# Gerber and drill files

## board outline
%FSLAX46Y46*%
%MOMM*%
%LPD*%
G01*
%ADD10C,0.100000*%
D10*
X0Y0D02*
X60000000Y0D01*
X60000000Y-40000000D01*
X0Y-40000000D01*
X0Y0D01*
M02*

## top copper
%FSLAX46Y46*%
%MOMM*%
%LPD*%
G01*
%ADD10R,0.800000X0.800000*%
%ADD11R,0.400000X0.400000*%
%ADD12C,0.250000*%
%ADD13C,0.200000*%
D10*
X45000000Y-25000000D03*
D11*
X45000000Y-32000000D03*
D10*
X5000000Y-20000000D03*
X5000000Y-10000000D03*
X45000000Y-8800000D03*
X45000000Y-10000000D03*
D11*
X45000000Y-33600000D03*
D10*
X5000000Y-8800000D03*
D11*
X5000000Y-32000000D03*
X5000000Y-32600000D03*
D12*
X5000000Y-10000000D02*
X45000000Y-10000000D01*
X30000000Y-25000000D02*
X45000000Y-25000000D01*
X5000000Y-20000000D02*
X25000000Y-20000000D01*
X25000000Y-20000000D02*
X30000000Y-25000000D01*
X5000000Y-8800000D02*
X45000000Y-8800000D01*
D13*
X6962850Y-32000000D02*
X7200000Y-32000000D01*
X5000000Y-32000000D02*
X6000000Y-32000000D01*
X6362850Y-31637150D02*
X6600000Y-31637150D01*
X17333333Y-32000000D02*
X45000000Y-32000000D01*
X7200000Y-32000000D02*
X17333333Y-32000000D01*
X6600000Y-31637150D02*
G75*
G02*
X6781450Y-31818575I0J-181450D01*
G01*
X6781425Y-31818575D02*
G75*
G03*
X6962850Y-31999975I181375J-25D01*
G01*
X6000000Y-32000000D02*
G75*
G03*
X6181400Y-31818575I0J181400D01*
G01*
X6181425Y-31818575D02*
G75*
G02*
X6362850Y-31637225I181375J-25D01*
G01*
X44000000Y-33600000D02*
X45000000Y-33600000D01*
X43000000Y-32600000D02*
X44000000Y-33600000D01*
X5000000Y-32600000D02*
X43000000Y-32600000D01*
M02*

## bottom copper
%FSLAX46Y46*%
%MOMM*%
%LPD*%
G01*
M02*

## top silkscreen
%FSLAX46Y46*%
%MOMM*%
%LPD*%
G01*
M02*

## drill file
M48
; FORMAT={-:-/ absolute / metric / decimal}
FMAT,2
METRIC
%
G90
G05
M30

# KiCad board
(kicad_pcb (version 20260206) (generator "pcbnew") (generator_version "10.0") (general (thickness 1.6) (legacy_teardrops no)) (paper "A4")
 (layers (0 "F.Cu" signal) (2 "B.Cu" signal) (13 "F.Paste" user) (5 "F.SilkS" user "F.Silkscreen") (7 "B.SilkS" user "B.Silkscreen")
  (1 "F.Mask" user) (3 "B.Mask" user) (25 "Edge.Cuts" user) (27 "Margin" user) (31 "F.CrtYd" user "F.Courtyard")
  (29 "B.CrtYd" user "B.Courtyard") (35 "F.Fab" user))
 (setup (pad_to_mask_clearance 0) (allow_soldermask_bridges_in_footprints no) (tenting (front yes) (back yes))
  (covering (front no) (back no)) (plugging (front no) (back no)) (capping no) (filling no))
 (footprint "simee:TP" (layer "F.Cu") (at 45 25)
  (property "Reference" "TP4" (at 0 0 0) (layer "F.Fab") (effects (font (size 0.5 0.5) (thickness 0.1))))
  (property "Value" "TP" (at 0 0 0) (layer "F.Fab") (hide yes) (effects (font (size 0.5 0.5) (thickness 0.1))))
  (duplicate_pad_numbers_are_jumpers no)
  (pad "1" smd rect (at 0 0) (size 0.8 0.8) (layers "F.Cu" "F.Mask") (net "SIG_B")))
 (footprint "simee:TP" (layer "F.Cu") (at 45 32)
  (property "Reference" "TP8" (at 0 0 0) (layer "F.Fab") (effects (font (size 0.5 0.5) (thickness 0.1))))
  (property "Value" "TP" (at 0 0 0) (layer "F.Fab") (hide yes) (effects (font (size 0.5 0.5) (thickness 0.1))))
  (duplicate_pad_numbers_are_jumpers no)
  (pad "1" smd rect (at 0 0) (size 0.4 0.4) (layers "F.Cu" "F.Mask") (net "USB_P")))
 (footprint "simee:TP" (layer "F.Cu") (at 5 20)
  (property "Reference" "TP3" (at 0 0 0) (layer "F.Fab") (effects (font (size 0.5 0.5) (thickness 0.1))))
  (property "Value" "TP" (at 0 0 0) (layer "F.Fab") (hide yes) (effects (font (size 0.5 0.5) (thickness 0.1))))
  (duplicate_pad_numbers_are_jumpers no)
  (pad "1" smd rect (at 0 0) (size 0.8 0.8) (layers "F.Cu" "F.Mask") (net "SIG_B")))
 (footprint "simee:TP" (layer "F.Cu") (at 5 10)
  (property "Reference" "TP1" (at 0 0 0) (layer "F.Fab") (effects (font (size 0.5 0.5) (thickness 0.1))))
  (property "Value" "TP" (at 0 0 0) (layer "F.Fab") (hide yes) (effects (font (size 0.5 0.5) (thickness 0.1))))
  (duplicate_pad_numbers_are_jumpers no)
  (pad "1" smd rect (at 0 0) (size 0.8 0.8) (layers "F.Cu" "F.Mask") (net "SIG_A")))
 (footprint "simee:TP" (layer "F.Cu") (at 45 8.8)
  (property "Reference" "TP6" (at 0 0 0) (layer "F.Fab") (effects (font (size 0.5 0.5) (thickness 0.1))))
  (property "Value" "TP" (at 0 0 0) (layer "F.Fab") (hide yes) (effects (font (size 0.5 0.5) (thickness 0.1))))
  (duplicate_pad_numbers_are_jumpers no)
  (pad "1" smd rect (at 0 0) (size 0.8 0.8) (layers "F.Cu" "F.Mask") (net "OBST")))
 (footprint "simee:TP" (layer "F.Cu") (at 45 10)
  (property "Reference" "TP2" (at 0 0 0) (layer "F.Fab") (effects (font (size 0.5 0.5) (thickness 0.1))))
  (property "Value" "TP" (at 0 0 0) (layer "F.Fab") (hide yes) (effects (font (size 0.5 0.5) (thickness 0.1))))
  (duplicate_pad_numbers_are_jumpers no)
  (pad "1" smd rect (at 0 0) (size 0.8 0.8) (layers "F.Cu" "F.Mask") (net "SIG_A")))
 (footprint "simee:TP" (layer "F.Cu") (at 45 33.6)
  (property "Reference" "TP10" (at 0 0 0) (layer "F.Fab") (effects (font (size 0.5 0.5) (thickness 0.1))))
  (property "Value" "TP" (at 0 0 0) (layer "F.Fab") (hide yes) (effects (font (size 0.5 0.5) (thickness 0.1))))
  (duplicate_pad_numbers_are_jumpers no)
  (pad "1" smd rect (at 0 0) (size 0.4 0.4) (layers "F.Cu" "F.Mask") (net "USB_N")))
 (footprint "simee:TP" (layer "F.Cu") (at 5 8.8)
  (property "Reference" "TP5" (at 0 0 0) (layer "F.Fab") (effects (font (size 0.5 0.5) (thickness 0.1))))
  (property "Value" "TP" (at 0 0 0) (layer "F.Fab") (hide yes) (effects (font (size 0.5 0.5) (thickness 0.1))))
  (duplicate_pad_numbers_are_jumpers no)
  (pad "1" smd rect (at 0 0) (size 0.8 0.8) (layers "F.Cu" "F.Mask") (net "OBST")))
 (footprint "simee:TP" (layer "F.Cu") (at 5 32)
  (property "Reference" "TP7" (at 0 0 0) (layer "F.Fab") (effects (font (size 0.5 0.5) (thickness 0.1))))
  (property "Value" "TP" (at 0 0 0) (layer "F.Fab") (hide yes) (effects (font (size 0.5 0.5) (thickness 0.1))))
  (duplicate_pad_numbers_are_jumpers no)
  (pad "1" smd rect (at 0 0) (size 0.4 0.4) (layers "F.Cu" "F.Mask") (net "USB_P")))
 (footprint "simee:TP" (layer "F.Cu") (at 5 32.6)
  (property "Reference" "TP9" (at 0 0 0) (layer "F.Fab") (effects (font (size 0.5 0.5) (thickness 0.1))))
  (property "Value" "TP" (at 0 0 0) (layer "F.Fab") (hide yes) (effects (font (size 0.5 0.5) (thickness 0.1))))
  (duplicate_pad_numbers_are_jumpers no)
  (pad "1" smd rect (at 0 0) (size 0.4 0.4) (layers "F.Cu" "F.Mask") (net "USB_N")))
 (gr_rect (start 0 0) (end 60 40) (stroke (width 0.1) (type default)) (fill no) (layer "Edge.Cuts"))
 (segment (start 5 10) (end 45 10) (width 0.25) (layer "F.Cu") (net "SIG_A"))
 (segment (start 30 25) (end 45 25) (width 0.25) (layer "F.Cu") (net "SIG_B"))
 (segment (start 5 20) (end 25 20) (width 0.25) (layer "F.Cu") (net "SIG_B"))
 (segment (start 25 20) (end 30 25) (width 0.25) (layer "F.Cu") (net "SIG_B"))
 (segment (start 5 8.8) (end 45 8.8) (width 0.25) (layer "F.Cu") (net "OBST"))
 (segment (start 6.96285 32) (end 7.2 32) (width 0.2) (layer "F.Cu") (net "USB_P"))
 (segment (start 5 32) (end 6 32) (width 0.2) (layer "F.Cu") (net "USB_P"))
 (segment (start 6.36285 31.63715) (end 6.6 31.63715) (width 0.2) (layer "F.Cu") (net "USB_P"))
 (segment (start 17.333333 32) (end 45 32) (width 0.2) (layer "F.Cu") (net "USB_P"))
 (segment (start 7.2 32) (end 17.333333 32) (width 0.2) (layer "F.Cu") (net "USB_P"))
 (arc (start 6.6 31.63715) (mid 6.728287 31.690288) (end 6.781425 31.818575) (width 0.2) (layer "F.Cu") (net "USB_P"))
 (arc (start 6.781425 31.818575) (mid 6.834563 31.946862) (end 6.96285 32) (width 0.2) (layer "F.Cu") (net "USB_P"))
 (arc (start 6 32) (mid 6.128287 31.946862) (end 6.181425 31.818575) (width 0.2) (layer "F.Cu") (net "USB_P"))
 (arc (start 6.181425 31.818575) (mid 6.234563 31.690288) (end 6.36285 31.63715) (width 0.2) (layer "F.Cu") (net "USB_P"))
 (segment (start 44 33.6) (end 45 33.6) (width 0.2) (layer "F.Cu") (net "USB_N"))
 (segment (start 43 32.6) (end 44 33.6) (width 0.2) (layer "F.Cu") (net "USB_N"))
 (segment (start 5 32.6) (end 43 32.6) (width 0.2) (layer "F.Cu") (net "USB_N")))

